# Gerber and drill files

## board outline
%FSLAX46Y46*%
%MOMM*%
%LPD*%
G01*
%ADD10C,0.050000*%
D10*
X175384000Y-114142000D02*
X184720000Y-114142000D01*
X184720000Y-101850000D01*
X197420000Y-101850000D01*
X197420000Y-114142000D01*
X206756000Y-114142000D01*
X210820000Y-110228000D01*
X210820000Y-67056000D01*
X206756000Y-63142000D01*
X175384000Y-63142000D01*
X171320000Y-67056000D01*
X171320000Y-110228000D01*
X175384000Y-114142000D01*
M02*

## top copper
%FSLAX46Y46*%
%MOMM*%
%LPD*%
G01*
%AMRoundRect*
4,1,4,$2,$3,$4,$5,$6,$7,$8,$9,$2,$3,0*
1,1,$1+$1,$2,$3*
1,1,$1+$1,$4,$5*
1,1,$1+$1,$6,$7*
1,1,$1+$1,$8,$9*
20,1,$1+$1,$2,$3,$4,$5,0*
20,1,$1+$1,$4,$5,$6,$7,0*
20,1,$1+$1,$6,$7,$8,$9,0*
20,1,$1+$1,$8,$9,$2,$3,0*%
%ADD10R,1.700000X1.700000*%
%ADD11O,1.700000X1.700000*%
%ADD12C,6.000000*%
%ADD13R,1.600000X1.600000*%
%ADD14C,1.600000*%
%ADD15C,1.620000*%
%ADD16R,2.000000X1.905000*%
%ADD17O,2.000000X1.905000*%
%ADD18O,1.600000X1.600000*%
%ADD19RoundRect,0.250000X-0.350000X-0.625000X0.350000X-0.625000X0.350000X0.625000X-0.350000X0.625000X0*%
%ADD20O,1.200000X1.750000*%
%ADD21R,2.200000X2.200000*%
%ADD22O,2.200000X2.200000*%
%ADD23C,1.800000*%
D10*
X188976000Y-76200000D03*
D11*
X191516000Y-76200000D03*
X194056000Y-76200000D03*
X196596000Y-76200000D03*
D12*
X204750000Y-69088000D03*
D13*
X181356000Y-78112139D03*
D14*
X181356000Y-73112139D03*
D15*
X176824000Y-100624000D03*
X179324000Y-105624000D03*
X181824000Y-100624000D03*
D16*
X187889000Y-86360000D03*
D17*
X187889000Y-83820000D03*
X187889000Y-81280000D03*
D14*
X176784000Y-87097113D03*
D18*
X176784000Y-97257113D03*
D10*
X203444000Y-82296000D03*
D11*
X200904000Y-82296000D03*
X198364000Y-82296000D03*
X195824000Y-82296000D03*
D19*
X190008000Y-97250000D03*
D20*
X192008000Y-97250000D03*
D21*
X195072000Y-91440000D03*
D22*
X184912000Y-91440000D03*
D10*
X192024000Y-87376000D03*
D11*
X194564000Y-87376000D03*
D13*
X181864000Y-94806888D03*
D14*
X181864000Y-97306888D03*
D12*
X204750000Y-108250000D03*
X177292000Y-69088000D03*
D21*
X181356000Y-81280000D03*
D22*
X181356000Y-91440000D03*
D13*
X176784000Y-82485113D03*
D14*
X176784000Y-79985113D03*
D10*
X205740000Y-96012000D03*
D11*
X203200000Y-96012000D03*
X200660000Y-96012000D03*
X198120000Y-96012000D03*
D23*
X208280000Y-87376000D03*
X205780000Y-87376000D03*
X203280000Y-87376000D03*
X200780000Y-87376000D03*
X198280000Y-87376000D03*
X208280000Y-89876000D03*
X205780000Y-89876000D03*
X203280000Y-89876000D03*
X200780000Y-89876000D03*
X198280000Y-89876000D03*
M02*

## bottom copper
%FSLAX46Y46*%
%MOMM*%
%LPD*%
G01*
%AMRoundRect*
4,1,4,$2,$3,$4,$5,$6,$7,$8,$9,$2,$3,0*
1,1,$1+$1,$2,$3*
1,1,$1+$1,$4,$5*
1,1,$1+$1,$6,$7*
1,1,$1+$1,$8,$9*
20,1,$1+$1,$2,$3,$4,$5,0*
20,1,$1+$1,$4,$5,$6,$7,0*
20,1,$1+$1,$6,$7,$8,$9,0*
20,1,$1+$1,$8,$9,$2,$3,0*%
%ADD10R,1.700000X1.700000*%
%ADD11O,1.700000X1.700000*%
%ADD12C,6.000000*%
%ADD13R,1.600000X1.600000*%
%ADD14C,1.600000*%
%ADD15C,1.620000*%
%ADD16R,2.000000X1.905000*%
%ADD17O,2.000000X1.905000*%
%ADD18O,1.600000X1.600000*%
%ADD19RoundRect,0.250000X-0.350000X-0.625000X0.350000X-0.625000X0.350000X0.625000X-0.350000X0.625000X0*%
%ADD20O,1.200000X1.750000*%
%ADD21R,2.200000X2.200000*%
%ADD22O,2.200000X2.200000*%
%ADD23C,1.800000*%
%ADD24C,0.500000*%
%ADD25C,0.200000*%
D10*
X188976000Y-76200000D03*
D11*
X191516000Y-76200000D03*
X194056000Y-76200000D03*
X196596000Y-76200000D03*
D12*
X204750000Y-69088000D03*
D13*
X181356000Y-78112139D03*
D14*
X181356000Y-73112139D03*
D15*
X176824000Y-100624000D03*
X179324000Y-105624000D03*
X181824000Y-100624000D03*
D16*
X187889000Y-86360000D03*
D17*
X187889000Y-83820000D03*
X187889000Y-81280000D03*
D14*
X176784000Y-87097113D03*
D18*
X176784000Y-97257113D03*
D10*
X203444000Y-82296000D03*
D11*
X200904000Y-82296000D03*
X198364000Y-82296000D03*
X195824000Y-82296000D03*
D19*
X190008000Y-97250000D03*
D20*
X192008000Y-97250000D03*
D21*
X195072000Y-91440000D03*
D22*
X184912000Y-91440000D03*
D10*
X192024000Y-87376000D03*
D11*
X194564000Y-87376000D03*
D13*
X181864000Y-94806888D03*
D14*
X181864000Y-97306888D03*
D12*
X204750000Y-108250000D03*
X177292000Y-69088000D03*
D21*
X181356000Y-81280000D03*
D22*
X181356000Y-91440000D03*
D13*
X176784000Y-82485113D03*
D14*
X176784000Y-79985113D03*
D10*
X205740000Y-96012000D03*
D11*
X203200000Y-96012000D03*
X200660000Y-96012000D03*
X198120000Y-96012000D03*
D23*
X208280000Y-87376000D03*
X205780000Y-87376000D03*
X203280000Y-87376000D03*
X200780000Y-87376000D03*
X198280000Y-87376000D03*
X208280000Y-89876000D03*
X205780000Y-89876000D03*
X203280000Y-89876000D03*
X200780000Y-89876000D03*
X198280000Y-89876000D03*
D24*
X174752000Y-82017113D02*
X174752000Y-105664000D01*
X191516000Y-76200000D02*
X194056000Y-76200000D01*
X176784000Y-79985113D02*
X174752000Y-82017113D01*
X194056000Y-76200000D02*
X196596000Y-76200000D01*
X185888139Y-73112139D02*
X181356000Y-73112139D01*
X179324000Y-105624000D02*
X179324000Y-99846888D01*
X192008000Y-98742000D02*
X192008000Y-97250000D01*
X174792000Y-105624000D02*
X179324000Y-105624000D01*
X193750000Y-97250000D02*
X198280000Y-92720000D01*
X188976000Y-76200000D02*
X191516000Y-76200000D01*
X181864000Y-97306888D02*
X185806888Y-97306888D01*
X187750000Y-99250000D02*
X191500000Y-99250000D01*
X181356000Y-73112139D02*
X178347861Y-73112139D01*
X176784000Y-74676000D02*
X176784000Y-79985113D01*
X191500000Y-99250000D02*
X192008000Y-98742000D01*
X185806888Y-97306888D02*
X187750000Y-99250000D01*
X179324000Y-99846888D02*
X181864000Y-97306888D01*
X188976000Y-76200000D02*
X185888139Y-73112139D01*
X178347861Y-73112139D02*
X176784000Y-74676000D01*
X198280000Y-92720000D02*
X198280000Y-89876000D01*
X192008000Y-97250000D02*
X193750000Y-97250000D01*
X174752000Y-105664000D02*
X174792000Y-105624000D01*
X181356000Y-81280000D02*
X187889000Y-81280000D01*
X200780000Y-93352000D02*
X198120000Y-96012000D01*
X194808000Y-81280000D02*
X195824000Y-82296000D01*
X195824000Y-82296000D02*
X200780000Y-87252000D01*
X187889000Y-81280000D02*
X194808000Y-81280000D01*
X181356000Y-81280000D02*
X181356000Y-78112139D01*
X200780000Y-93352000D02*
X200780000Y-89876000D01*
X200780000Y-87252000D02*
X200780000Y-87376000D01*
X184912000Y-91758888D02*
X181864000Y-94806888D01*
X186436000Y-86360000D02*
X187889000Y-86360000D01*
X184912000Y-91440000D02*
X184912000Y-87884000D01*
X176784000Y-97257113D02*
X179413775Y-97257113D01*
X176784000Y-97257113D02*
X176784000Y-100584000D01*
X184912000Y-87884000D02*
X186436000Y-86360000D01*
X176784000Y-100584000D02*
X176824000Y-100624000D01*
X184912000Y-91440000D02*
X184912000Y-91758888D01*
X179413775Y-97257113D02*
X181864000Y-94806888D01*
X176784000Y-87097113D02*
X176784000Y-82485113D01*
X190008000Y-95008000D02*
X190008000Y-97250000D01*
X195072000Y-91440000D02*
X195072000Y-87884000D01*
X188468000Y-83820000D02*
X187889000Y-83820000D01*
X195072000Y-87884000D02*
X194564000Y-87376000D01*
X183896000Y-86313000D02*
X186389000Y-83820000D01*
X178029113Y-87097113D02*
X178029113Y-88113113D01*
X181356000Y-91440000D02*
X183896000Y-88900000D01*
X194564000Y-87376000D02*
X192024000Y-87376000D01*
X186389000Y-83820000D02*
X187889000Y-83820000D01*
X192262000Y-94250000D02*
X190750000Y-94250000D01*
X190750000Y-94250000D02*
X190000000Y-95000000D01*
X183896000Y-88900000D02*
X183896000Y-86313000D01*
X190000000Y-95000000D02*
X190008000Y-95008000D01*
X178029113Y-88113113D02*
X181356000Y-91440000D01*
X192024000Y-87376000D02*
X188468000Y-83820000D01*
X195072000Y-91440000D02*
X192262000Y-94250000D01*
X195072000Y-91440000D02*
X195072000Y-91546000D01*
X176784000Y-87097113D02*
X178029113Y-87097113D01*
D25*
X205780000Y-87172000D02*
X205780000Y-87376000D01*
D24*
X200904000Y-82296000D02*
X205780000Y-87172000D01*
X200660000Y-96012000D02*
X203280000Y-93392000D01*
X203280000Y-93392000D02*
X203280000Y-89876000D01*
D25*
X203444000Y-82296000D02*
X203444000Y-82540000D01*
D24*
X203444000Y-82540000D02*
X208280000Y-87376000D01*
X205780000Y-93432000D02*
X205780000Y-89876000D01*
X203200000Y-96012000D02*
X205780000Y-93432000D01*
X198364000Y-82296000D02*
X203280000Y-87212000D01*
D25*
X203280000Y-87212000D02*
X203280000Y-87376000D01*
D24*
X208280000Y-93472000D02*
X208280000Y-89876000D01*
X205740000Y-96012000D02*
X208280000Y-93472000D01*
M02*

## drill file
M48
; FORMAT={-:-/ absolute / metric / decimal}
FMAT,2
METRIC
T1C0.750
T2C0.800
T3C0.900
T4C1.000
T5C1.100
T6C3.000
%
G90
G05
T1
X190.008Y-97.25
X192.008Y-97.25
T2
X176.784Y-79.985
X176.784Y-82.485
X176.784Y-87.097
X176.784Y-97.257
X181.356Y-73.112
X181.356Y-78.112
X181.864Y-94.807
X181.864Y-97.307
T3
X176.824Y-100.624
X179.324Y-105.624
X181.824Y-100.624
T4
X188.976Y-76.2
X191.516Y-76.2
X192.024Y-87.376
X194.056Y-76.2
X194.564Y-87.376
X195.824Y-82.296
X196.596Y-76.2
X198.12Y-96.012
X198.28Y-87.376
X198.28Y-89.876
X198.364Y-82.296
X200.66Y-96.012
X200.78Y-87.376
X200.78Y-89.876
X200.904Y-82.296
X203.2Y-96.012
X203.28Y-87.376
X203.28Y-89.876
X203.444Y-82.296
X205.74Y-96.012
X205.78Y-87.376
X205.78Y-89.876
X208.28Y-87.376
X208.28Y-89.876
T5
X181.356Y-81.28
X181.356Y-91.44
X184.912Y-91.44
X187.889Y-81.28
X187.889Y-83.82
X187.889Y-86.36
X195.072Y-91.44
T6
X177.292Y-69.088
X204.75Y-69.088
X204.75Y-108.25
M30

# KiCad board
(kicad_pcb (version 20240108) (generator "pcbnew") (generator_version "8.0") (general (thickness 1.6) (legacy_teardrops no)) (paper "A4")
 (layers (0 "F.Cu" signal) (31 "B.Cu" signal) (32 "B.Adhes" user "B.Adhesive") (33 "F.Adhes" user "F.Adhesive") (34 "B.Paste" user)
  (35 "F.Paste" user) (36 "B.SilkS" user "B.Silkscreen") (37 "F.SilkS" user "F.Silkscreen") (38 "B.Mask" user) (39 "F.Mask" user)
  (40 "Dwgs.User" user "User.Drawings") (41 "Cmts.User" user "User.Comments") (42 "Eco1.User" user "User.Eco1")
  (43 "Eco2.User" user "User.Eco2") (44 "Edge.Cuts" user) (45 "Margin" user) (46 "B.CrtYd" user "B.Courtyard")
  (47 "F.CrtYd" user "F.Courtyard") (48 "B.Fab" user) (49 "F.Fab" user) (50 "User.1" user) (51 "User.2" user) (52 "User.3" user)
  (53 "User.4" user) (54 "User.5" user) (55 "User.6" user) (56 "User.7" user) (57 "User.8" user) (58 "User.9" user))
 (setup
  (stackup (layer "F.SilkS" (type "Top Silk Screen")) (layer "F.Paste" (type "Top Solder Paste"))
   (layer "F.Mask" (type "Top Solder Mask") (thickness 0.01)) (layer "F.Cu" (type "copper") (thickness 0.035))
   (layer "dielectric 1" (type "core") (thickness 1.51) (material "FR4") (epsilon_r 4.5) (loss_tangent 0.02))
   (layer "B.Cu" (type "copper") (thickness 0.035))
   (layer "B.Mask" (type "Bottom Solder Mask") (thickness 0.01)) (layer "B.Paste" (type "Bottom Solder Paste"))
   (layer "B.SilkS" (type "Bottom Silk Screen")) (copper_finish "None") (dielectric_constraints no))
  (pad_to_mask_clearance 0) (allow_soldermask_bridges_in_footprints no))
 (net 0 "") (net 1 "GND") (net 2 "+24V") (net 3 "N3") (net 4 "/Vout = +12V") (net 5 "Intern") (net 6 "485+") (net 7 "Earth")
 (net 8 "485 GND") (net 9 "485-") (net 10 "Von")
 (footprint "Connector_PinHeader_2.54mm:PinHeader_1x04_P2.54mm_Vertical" (layer "F.Cu") (at 188.976 76.2 90)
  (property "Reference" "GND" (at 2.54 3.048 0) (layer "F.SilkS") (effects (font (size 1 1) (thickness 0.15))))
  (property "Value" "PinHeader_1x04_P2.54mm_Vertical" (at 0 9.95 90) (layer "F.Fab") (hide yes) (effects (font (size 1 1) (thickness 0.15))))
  (pad "1" thru_hole rect (at 0 0 90) (size 1.7 1.7) (drill 1) (layers "*.Cu" "*.Mask") (remove_unused_layers no) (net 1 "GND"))
  (pad "2" thru_hole oval (at 0 2.54 90) (size 1.7 1.7) (drill 1) (layers "*.Cu" "*.Mask") (remove_unused_layers no) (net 1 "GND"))
  (pad "3" thru_hole oval (at 0 5.08 90) (size 1.7 1.7) (drill 1) (layers "*.Cu" "*.Mask") (remove_unused_layers no) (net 1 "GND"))
  (pad "4" thru_hole oval (at 0 7.62 90) (size 1.7 1.7) (drill 1) (layers "*.Cu" "*.Mask") (remove_unused_layers no) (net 1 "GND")))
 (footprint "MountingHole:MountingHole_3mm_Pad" (layer "F.Cu") (at 204.75 69.088)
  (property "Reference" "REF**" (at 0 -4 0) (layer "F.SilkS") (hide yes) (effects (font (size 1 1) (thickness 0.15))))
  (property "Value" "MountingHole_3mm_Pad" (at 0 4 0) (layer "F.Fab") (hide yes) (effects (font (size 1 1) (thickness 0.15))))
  (pad "1" thru_hole circle (at 0 0) (size 6 6) (drill 3) (layers "*.Cu" "*.Mask") (remove_unused_layers no)))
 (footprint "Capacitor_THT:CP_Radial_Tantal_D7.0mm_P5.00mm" (layer "F.Cu") (at 181.356 78.112139 90)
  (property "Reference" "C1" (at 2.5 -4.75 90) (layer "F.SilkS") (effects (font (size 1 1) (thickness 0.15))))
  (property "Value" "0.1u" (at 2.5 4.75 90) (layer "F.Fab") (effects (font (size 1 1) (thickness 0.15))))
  (pad "1" thru_hole rect (at 0 0 90) (size 1.6 1.6) (drill 0.8) (layers "*.Cu" "*.Mask") (remove_unused_layers no) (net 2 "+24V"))
  (pad "2" thru_hole circle (at 5 0 90) (size 1.6 1.6) (drill 0.8) (layers "*.Cu" "*.Mask") (remove_unused_layers no) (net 1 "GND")))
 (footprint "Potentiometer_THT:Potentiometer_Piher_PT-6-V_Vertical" (layer "F.Cu") (at 176.824 100.624 -90)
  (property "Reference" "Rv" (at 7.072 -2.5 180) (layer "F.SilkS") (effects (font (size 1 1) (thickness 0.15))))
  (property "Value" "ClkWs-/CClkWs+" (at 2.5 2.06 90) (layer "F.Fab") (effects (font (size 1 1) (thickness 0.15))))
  (pad "1" thru_hole circle (at 0 0 270) (size 1.62 1.62) (drill 0.9) (layers "*.Cu" "*.Mask") (remove_unused_layers no) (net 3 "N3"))
  (pad "2" thru_hole circle (at 5 -2.5 270) (size 1.62 1.62) (drill 0.9) (layers "*.Cu" "*.Mask") (remove_unused_layers no) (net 1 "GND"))
  (pad "3" thru_hole circle (at 0 -5 270) (size 1.62 1.62) (drill 0.9) (layers "*.Cu" "*.Mask") (remove_unused_layers no)))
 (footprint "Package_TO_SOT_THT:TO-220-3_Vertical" (layer "F.Cu") (at 187.889 86.36 90)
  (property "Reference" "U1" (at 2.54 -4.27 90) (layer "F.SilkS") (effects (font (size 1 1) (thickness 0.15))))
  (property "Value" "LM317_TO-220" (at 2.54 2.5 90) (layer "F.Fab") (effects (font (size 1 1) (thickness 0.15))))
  (pad "1" thru_hole rect (at 0 0 90) (size 1.905 2) (drill 1.1) (layers "*.Cu" "*.Mask") (remove_unused_layers no) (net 3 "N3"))
  (pad "2" thru_hole oval (at 2.54 0 90) (size 1.905 2) (drill 1.1) (layers "*.Cu" "*.Mask") (remove_unused_layers no)
   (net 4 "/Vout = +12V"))
  (pad "3" thru_hole oval (at 5.08 0 90) (size 1.905 2) (drill 1.1) (layers "*.Cu" "*.Mask") (remove_unused_layers no) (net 2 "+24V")))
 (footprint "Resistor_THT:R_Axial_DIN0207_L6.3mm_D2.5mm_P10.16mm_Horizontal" (layer "F.Cu") (at 176.784 87.097113 -90)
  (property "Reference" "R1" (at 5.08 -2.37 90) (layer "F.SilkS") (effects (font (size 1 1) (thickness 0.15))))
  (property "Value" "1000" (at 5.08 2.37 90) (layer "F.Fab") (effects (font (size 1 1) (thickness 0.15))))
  (pad "1" thru_hole circle (at 0 0 270) (size 1.6 1.6) (drill 0.8) (layers "*.Cu" "*.Mask") (remove_unused_layers no)
   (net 4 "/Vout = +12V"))
  (pad "2" thru_hole oval (at 10.16 0 270) (size 1.6 1.6) (drill 0.8) (layers "*.Cu" "*.Mask") (remove_unused_layers no) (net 3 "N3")))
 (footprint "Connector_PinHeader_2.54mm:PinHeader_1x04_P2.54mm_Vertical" (layer "F.Cu") (at 203.444 82.296 -90)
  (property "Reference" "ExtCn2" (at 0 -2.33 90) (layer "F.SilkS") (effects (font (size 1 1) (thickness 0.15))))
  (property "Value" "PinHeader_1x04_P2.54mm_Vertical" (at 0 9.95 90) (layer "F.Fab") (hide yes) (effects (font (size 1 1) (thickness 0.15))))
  (pad "1" thru_hole rect (at 0 0 270) (size 1.7 1.7) (drill 1) (layers "*.Cu" "*.Mask" "B.Paste") (remove_unused_layers no)
   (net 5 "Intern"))
  (pad "2" thru_hole oval (at 0 2.54 270) (size 1.7 1.7) (drill 1) (layers "*.Cu" "*.Mask") (remove_unused_layers no) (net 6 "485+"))
  (pad "3" thru_hole oval (at 0 5.08 270) (size 1.7 1.7) (drill 1) (layers "*.Cu" "*.Mask" "Eco1.User") (remove_unused_layers no)
   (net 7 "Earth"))
  (pad "4" thru_hole oval (at 0 7.62 270) (size 1.7 1.7) (drill 1) (layers "*.Cu" "*.Mask") (remove_unused_layers no) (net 2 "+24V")))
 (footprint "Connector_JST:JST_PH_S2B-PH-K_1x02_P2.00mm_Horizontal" (layer "F.Cu") (at 190.008 97.25)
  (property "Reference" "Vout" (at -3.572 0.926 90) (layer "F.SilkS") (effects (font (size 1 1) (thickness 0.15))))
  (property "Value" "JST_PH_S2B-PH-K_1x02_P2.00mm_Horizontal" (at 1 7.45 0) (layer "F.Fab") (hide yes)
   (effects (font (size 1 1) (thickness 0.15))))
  (pad "1" thru_hole roundrect (at 0 0) (size 1.2 1.75) (drill 0.75) (layers "*.Cu" "*.Mask") (remove_unused_layers no)
   (roundrect_rratio 0.208333) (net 4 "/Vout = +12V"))
  (pad "2" thru_hole oval (at 2 0) (size 1.2 1.75) (drill 0.75) (layers "*.Cu" "*.Mask") (remove_unused_layers no) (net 1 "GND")))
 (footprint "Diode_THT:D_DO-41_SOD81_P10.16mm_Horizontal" (layer "F.Cu") (at 195.072 91.44 180)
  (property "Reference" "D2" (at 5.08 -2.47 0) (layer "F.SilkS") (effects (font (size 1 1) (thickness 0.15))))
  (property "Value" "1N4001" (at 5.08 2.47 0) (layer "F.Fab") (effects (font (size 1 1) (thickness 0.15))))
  (pad "1" thru_hole rect (at 0 0 180) (size 2.2 2.2) (drill 1.1) (layers "*.Cu" "*.Mask") (remove_unused_layers no) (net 4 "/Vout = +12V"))
  (pad "2" thru_hole oval (at 10.16 0 180) (size 2.2 2.2) (drill 1.1) (layers "*.Cu" "*.Mask") (remove_unused_layers no) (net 3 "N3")))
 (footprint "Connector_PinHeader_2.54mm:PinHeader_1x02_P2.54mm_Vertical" (layer "F.Cu") (at 192.024 87.376 90)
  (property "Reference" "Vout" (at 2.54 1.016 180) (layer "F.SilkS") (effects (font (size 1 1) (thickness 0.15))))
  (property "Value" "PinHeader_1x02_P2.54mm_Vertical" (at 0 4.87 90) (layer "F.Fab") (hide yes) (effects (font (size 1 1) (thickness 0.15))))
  (pad "" thru_hole rect (at 0 0 90) (size 1.7 1.7) (drill 1) (layers "*.Cu" "*.Mask") (remove_unused_layers no) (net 4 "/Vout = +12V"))
  (pad "2" thru_hole oval (at 0 2.54 90) (size 1.7 1.7) (drill 1) (layers "*.Cu" "*.Mask") (remove_unused_layers no) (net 4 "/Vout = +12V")))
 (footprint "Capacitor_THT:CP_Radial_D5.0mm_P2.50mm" (layer "F.Cu") (at 181.864 94.806888 -90)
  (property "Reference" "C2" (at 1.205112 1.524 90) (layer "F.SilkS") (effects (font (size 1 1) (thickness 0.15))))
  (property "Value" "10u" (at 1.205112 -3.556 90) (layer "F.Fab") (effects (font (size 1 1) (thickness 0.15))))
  (pad "1" thru_hole rect (at 0 0 270) (size 1.6 1.6) (drill 0.8) (layers "*.Cu" "*.Mask") (remove_unused_layers no) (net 3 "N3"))
  (pad "2" thru_hole circle (at 2.5 0 270) (size 1.6 1.6) (drill 0.8) (layers "*.Cu" "*.Mask") (remove_unused_layers no) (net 1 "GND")))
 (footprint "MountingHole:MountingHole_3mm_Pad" (layer "F.Cu") (at 204.75 108.25)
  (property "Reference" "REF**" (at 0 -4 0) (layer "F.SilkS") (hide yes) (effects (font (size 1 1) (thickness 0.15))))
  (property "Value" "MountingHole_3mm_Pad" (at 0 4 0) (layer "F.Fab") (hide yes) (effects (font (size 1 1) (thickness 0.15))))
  (pad "1" thru_hole circle (at 0 0) (size 6 6) (drill 3) (layers "*.Cu" "*.Mask") (remove_unused_layers no)))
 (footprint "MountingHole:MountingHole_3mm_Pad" (layer "F.Cu") (at 177.292 69.088)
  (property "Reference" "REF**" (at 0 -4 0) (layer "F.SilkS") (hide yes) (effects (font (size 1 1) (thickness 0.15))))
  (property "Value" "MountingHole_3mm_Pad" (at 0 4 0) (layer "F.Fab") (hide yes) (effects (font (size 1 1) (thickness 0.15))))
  (pad "1" thru_hole circle (at 0 0) (size 6 6) (drill 3) (layers "*.Cu" "*.Mask") (remove_unused_layers no)))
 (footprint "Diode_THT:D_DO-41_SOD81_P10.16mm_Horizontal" (layer "F.Cu") (at 181.356 81.28 -90)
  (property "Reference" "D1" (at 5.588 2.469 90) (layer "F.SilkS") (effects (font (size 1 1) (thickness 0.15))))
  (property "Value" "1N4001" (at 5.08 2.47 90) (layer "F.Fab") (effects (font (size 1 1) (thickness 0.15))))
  (pad "1" thru_hole rect (at 0 0 270) (size 2.2 2.2) (drill 1.1) (layers "*.Cu" "*.Mask") (remove_unused_layers no) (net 2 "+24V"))
  (pad "2" thru_hole oval (at 10.16 0 270) (size 2.2 2.2) (drill 1.1) (layers "*.Cu" "*.Mask") (remove_unused_layers no)
   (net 4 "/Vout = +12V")))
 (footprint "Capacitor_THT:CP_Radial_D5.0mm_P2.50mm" (layer "F.Cu") (at 176.784 82.485113 90)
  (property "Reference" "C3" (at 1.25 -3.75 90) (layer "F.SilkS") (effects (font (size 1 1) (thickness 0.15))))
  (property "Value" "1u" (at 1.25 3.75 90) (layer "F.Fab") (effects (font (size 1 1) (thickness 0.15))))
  (pad "1" thru_hole rect (at 0 0 90) (size 1.6 1.6) (drill 0.8) (layers "*.Cu" "*.Mask") (remove_unused_layers no) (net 4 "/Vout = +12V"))
  (pad "2" thru_hole circle (at 2.5 0 90) (size 1.6 1.6) (drill 0.8) (layers "*.Cu" "*.Mask") (remove_unused_layers no) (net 1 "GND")))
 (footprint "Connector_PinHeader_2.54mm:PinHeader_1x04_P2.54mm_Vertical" (layer "F.Cu") (at 205.74 96.012 -90)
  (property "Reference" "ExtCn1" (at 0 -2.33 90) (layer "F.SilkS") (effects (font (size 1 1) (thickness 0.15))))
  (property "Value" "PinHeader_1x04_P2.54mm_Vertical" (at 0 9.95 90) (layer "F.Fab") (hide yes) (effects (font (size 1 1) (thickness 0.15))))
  (pad "1" thru_hole rect (at 0 0 270) (size 1.7 1.7) (drill 1) (layers "*.Cu" "*.Mask") (remove_unused_layers no) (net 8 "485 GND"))
  (pad "2" thru_hole oval (at 0 2.54 270) (size 1.7 1.7) (drill 1) (layers "*.Cu" "*.Mask") (remove_unused_layers no) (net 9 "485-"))
  (pad "3" thru_hole oval (at 0 5.08 270) (size 1.7 1.7) (drill 1) (layers "*.Cu" "*.Mask") (remove_unused_layers no) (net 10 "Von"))
  (pad "4" thru_hole oval (at 0 7.62 270) (size 1.7 1.7) (drill 1) (layers "*.Cu" "*.Mask") (remove_unused_layers no) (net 2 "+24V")))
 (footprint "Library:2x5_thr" (layer "B.Cu") (at 208.28 87.376 180)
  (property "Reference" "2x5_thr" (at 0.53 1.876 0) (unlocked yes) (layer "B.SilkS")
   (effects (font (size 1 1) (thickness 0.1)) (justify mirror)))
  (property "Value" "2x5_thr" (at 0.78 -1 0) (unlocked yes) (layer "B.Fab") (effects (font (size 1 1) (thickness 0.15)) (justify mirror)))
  (pad "1" thru_hole circle (at 0 0 180) (size 1.8 1.8) (drill 1) (layers "*.Cu" "*.Mask") (remove_unused_layers no) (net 5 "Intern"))
  (pad "2" thru_hole circle (at 2.5 0 180) (size 1.8 1.8) (drill 1) (layers "*.Cu" "*.Mask") (remove_unused_layers no) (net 6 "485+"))
  (pad "3" thru_hole circle (at 5 0 180) (size 1.8 1.8) (drill 1) (layers "*.Cu" "*.Mask") (remove_unused_layers no) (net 7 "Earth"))
  (pad "4" thru_hole circle (at 7.5 0 180) (size 1.8 1.8) (drill 1) (layers "*.Cu" "*.Mask") (remove_unused_layers no) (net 2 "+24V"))
  (pad "5" thru_hole circle (at 10 0 180) (size 1.8 1.8) (drill 1) (layers "*.Cu" "*.Mask") (remove_unused_layers no) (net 1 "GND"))
  (pad "6" thru_hole circle (at 0 -2.5 180) (size 1.8 1.8) (drill 1) (layers "*.Cu" "*.Mask") (remove_unused_layers no) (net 8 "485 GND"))
  (pad "7" thru_hole circle (at 2.5 -2.5 180) (size 1.8 1.8) (drill 1) (layers "*.Cu" "*.Mask") (remove_unused_layers no) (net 9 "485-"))
  (pad "8" thru_hole circle (at 5 -2.5 180) (size 1.8 1.8) (drill 1) (layers "*.Cu" "*.Mask") (remove_unused_layers no) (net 10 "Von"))
  (pad "9" thru_hole circle (at 7.5 -2.5 180) (size 1.8 1.8) (drill 1) (layers "*.Cu" "*.Mask") (remove_unused_layers no) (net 2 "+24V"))
  (pad "10" thru_hole circle (at 10 -2.5 180) (size 1.8 1.8) (drill 1) (layers "*.Cu" "*.Mask") (remove_unused_layers no) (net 1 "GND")))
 (gr_poly
  (pts (xy 175.384 114.142) (xy 184.72 114.142) (xy 184.72 101.85) (xy 197.42 101.85) (xy 197.42 114.142) (xy 206.756 114.142)
   (xy 210.82 110.228) (xy 210.82 67.056) (xy 206.756 63.142) (xy 175.384 63.142) (xy 171.32 67.056) (xy 171.32 110.228))
  (stroke (width 0.05) (type solid)) (fill none) (layer "Edge.Cuts"))
 (segment (start 174.752 82.017113) (end 174.752 105.664) (width 0.5) (layer "B.Cu") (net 1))
 (segment (start 191.516 76.2) (end 194.056 76.2) (width 0.5) (layer "B.Cu") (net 1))
 (segment (start 176.784 79.985113) (end 174.752 82.017113) (width 0.5) (layer "B.Cu") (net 1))
 (segment (start 194.056 76.2) (end 196.596 76.2) (width 0.5) (layer "B.Cu") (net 1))
 (segment (start 185.888139 73.112139) (end 181.356 73.112139) (width 0.5) (layer "B.Cu") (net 1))
 (segment (start 179.324 105.624) (end 179.324 99.846888) (width 0.5) (layer "B.Cu") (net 1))
 (segment (start 192.008 98.742) (end 192.008 97.25) (width 0.5) (layer "B.Cu") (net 1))
 (segment (start 174.792 105.624) (end 179.324 105.624) (width 0.5) (layer "B.Cu") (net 1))
 (segment (start 193.75 97.25) (end 198.28 92.72) (width 0.5) (layer "B.Cu") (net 1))
 (segment (start 188.976 76.2) (end 191.516 76.2) (width 0.5) (layer "B.Cu") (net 1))
 (segment (start 181.864 97.306888) (end 185.806888 97.306888) (width 0.5) (layer "B.Cu") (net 1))
 (segment (start 187.75 99.25) (end 191.5 99.25) (width 0.5) (layer "B.Cu") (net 1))
 (segment (start 181.356 73.112139) (end 178.347861 73.112139) (width 0.5) (layer "B.Cu") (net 1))
 (segment (start 176.784 74.676) (end 176.784 79.985113) (width 0.5) (layer "B.Cu") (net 1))
 (segment (start 191.5 99.25) (end 192.008 98.742) (width 0.5) (layer "B.Cu") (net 1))
 (segment (start 185.806888 97.306888) (end 187.75 99.25) (width 0.5) (layer "B.Cu") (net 1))
 (segment (start 179.324 99.846888) (end 181.864 97.306888) (width 0.5) (layer "B.Cu") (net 1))
 (segment (start 188.976 76.2) (end 185.888139 73.112139) (width 0.5) (layer "B.Cu") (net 1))
 (segment (start 178.347861 73.112139) (end 176.784 74.676) (width 0.5) (layer "B.Cu") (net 1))
 (segment (start 198.28 92.72) (end 198.28 89.876) (width 0.5) (layer "B.Cu") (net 1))
 (segment (start 192.008 97.25) (end 193.75 97.25) (width 0.5) (layer "B.Cu") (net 1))
 (segment (start 174.752 105.664) (end 174.792 105.624) (width 0.5) (layer "B.Cu") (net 1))
 (segment (start 181.356 81.28) (end 187.889 81.28) (width 0.5) (layer "B.Cu") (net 2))
 (segment (start 200.78 93.352) (end 198.12 96.012) (width 0.5) (layer "B.Cu") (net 2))
 (segment (start 194.808 81.28) (end 195.824 82.296) (width 0.5) (layer "B.Cu") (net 2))
 (segment (start 195.824 82.296) (end 200.78 87.252) (width 0.5) (layer "B.Cu") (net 2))
 (segment (start 187.889 81.28) (end 194.808 81.28) (width 0.5) (layer "B.Cu") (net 2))
 (segment (start 181.356 81.28) (end 181.356 78.112139) (width 0.5) (layer "B.Cu") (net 2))
 (segment (start 200.78 93.352) (end 200.78 89.876) (width 0.5) (layer "B.Cu") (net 2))
 (segment (start 200.78 87.252) (end 200.78 87.376) (width 0.5) (layer "B.Cu") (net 2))
 (segment (start 184.912 91.758888) (end 181.864 94.806888) (width 0.5) (layer "B.Cu") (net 3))
 (segment (start 186.436 86.36) (end 187.889 86.36) (width 0.5) (layer "B.Cu") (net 3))
 (segment (start 184.912 91.44) (end 184.912 87.884) (width 0.5) (layer "B.Cu") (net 3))
 (segment (start 176.784 97.257113) (end 179.413775 97.257113) (width 0.5) (layer "B.Cu") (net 3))
 (segment (start 176.784 97.257113) (end 176.784 100.584) (width 0.5) (layer "B.Cu") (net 3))
 (segment (start 184.912 87.884) (end 186.436 86.36) (width 0.5) (layer "B.Cu") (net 3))
 (segment (start 176.784 100.584) (end 176.824 100.624) (width 0.5) (layer "B.Cu") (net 3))
 (segment (start 184.912 91.44) (end 184.912 91.758888) (width 0.5) (layer "B.Cu") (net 3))
 (segment (start 179.413775 97.257113) (end 181.864 94.806888) (width 0.5) (layer "B.Cu") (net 3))
 (segment (start 176.784 87.097113) (end 176.784 82.485113) (width 0.5) (layer "B.Cu") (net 4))
 (segment (start 190.008 95.008) (end 190.008 97.25) (width 0.5) (layer "B.Cu") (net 4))
 (segment (start 195.072 91.44) (end 195.072 87.884) (width 0.5) (layer "B.Cu") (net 4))
 (segment (start 188.468 83.82) (end 187.889 83.82) (width 0.5) (layer "B.Cu") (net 4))
 (segment (start 195.072 87.884) (end 194.564 87.376) (width 0.5) (layer "B.Cu") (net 4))
 (segment (start 183.896 86.313) (end 186.389 83.82) (width 0.5) (layer "B.Cu") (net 4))
 (segment (start 178.029113 87.097113) (end 178.029113 88.113113) (width 0.5) (layer "B.Cu") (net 4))
 (segment (start 181.356 91.44) (end 183.896 88.9) (width 0.5) (layer "B.Cu") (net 4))
 (segment (start 194.564 87.376) (end 192.024 87.376) (width 0.5) (layer "B.Cu") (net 4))
 (segment (start 186.389 83.82) (end 187.889 83.82) (width 0.5) (layer "B.Cu") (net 4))
 (segment (start 192.262 94.25) (end 190.75 94.25) (width 0.5) (layer "B.Cu") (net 4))
 (segment (start 190.75 94.25) (end 190 95) (width 0.5) (layer "B.Cu") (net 4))
 (segment (start 183.896 88.9) (end 183.896 86.313) (width 0.5) (layer "B.Cu") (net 4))
 (segment (start 190 95) (end 190.008 95.008) (width 0.5) (layer "B.Cu") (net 4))
 (segment (start 178.029113 88.113113) (end 181.356 91.44) (width 0.5) (layer "B.Cu") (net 4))
 (segment (start 192.024 87.376) (end 188.468 83.82) (width 0.5) (layer "B.Cu") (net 4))
 (segment (start 195.072 91.44) (end 192.262 94.25) (width 0.5) (layer "B.Cu") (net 4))
 (segment (start 195.072 91.44) (end 195.072 91.546) (width 0.5) (layer "B.Cu") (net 4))
 (segment (start 176.784 87.097113) (end 178.029113 87.097113) (width 0.5) (layer "B.Cu") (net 4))
 (segment (start 205.78 87.172) (end 205.78 87.376) (width 0.2) (layer "B.Cu") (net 6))
 (segment (start 200.904 82.296) (end 205.78 87.172) (width 0.5) (layer "B.Cu") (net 6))
 (segment (start 200.66 96.012) (end 203.28 93.392) (width 0.5) (layer "B.Cu") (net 10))
 (segment (start 203.28 93.392) (end 203.28 89.876) (width 0.5) (layer "B.Cu") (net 10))
 (segment (start 203.444 82.296) (end 203.444 82.54) (width 0.2) (layer "B.Cu") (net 5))
 (segment (start 203.444 82.54) (end 208.28 87.376) (width 0.5) (layer "B.Cu") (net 5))
 (segment (start 205.78 93.432) (end 205.78 89.876) (width 0.5) (layer "B.Cu") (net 9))
 (segment (start 203.2 96.012) (end 205.78 93.432) (width 0.5) (layer "B.Cu") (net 9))
 (segment (start 198.364 82.296) (end 203.28 87.212) (width 0.5) (layer "B.Cu") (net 7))
 (segment (start 203.28 87.212) (end 203.28 87.376) (width 0.2) (layer "B.Cu") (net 7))
 (segment (start 208.28 93.472) (end 208.28 89.876) (width 0.5) (layer "B.Cu") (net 8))
 (segment (start 205.74 96.012) (end 208.28 93.472) (width 0.5) (layer "B.Cu") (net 8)))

